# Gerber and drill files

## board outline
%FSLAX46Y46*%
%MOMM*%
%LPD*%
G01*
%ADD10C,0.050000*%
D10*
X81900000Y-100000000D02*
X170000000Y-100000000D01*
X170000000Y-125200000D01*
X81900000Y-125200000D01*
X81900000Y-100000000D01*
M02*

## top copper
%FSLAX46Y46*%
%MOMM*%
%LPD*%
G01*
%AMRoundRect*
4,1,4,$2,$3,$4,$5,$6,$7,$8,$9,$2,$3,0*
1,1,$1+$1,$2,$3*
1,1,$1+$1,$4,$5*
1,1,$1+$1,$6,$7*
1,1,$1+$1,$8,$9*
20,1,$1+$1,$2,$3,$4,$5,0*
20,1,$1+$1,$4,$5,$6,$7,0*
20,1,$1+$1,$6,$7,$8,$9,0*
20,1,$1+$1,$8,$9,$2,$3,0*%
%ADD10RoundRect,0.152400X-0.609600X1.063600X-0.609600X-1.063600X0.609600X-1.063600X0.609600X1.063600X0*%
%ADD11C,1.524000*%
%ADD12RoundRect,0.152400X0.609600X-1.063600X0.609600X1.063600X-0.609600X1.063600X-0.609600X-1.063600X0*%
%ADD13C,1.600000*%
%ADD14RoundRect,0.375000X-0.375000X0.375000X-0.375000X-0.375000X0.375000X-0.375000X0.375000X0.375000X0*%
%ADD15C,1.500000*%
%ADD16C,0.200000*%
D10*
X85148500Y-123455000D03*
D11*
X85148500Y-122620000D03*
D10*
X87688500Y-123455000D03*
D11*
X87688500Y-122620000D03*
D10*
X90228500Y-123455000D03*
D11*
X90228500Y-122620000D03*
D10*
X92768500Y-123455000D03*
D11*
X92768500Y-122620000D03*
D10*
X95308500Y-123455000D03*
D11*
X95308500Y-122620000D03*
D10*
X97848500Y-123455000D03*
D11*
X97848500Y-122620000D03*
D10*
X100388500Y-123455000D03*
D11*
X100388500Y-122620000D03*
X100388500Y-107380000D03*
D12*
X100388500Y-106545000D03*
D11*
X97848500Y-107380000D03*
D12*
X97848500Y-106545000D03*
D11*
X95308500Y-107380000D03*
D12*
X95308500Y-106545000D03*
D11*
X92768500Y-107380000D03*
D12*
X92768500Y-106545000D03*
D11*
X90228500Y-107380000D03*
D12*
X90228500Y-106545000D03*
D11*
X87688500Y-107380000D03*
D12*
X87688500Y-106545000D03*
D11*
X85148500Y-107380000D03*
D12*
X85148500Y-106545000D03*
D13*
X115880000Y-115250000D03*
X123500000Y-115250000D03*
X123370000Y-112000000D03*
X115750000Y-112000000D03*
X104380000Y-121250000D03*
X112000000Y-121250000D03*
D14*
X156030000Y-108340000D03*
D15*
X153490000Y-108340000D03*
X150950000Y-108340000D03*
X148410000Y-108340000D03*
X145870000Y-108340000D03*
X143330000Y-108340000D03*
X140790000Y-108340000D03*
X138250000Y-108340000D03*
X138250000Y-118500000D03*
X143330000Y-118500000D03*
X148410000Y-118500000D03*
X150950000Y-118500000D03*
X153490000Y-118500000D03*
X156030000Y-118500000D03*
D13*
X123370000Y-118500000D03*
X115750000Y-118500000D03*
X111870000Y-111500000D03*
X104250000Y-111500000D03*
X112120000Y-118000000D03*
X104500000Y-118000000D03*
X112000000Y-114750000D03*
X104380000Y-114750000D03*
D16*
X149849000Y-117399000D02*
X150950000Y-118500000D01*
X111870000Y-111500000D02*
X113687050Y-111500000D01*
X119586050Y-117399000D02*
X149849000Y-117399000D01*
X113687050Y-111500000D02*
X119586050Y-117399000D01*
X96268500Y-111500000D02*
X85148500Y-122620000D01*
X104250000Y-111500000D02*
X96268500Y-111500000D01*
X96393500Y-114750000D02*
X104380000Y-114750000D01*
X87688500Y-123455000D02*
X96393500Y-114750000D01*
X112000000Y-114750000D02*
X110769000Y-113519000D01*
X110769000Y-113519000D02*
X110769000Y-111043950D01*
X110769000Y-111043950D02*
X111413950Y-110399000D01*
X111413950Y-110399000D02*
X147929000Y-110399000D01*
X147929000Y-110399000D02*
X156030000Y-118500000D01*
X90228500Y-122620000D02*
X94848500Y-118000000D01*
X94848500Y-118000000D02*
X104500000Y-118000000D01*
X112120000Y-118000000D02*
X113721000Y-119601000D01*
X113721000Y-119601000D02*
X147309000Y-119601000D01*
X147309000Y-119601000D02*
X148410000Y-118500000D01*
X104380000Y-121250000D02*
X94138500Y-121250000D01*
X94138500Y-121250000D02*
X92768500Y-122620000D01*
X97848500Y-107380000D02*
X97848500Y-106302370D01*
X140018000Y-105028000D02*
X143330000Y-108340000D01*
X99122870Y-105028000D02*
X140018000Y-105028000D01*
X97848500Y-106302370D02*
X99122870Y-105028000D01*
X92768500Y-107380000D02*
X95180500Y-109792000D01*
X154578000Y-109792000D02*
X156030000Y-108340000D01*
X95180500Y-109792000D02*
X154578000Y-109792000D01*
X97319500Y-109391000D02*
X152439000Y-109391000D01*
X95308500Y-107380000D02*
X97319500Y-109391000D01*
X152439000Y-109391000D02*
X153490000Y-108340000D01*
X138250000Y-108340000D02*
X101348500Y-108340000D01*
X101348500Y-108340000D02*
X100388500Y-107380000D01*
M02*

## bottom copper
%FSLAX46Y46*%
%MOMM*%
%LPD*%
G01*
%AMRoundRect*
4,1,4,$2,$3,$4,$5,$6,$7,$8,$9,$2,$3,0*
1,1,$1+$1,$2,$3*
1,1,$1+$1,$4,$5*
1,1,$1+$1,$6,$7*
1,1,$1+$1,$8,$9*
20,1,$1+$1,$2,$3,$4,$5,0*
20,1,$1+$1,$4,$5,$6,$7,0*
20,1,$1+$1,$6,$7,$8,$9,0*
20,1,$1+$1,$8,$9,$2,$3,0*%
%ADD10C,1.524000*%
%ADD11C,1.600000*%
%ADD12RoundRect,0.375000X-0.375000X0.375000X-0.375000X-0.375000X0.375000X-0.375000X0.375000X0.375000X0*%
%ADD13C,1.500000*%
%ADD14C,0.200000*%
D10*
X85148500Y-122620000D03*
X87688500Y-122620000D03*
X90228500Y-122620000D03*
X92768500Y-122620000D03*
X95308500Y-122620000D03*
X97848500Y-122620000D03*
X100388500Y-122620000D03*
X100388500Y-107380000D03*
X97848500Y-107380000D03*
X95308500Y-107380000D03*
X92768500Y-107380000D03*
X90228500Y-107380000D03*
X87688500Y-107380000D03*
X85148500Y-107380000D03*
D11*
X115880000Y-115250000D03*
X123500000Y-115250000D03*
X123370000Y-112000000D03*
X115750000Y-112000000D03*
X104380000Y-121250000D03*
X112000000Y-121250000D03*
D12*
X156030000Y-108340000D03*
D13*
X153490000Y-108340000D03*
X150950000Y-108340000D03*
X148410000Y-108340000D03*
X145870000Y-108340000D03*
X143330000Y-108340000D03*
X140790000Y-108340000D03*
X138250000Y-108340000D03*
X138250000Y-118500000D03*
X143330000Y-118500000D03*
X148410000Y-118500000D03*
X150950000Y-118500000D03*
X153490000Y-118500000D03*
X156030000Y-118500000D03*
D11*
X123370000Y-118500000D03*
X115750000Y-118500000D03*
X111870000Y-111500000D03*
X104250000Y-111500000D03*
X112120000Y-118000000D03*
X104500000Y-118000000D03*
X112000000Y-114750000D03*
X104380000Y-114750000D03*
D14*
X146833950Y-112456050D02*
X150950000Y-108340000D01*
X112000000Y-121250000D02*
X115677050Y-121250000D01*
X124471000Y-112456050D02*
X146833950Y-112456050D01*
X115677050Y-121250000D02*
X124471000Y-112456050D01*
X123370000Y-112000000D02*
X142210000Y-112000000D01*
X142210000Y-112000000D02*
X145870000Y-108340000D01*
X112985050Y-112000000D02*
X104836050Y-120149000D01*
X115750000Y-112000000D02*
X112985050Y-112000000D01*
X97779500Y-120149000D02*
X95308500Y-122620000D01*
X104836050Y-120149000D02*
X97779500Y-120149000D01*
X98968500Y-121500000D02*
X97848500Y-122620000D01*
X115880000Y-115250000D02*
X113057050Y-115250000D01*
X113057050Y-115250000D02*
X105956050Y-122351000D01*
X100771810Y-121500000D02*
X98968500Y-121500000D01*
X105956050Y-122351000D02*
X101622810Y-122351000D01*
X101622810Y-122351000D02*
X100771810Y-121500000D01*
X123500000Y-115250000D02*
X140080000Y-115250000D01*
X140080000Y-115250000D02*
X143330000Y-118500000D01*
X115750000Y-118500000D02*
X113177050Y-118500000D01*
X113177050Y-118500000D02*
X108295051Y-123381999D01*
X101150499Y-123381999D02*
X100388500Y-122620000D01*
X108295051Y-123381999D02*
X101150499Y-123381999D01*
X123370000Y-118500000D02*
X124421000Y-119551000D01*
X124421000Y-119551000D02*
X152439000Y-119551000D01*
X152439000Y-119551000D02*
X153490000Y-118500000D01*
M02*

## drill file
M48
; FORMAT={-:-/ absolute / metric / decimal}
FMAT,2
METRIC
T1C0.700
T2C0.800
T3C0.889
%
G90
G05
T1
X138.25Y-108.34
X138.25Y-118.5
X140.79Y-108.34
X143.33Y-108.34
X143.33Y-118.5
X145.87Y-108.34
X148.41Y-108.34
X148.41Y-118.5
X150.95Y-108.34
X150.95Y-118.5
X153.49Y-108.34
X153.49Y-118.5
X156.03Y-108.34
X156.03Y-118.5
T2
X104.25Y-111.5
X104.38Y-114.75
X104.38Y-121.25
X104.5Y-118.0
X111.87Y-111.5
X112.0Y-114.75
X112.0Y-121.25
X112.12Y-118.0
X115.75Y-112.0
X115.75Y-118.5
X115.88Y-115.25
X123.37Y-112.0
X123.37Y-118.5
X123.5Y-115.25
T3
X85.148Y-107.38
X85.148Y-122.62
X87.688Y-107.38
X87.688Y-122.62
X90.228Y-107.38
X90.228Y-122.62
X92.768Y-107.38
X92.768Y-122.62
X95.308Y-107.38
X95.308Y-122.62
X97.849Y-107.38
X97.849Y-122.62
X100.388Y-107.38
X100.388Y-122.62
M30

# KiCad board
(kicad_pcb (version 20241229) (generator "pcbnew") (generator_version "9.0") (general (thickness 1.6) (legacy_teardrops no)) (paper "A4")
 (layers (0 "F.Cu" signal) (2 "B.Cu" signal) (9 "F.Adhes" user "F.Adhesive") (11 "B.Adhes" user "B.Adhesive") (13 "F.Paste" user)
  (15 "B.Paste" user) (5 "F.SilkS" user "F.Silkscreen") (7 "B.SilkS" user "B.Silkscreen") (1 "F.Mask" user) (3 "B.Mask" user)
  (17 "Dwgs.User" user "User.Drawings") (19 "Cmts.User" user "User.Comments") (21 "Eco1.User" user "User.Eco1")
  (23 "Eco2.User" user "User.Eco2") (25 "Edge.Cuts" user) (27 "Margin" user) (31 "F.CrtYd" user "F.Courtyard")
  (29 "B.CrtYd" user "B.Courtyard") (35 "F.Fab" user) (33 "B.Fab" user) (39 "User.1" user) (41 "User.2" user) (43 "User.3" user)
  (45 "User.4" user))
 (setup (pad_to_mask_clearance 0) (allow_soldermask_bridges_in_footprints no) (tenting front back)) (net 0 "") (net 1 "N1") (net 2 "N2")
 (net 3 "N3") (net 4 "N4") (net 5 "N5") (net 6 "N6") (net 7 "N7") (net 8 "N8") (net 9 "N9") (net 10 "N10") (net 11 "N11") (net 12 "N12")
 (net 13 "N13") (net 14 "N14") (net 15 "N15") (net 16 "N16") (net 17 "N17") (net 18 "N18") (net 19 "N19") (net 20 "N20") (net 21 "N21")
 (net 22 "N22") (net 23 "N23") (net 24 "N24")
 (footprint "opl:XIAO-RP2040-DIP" (layer "F.Cu") (at 92.7685 115 90)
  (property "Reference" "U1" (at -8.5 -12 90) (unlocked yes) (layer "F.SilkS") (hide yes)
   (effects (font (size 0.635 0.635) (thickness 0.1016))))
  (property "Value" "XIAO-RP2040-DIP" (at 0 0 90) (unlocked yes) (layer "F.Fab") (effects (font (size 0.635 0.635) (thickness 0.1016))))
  (pad "1" smd roundrect (at -8.455 -7.62 270) (size 2.432 1.524) (layers "F.Cu" "F.Mask") (roundrect_rratio 0.1) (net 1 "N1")
   (thermal_bridge_angle 45))
  (pad "1" thru_hole circle (at -7.62 -7.62 270) (size 1.524 1.524) (drill 0.889) (layers "*.Cu" "*.Mask") (remove_unused_layers no)
   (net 1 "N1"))
  (pad "2" smd roundrect (at -8.455 -5.08 270) (size 2.432 1.524) (layers "F.Cu" "F.Mask") (roundrect_rratio 0.1) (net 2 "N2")
   (thermal_bridge_angle 45))
  (pad "2" thru_hole circle (at -7.62 -5.08 270) (size 1.524 1.524) (drill 0.889) (layers "*.Cu" "*.Mask") (remove_unused_layers no)
   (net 2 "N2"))
  (pad "3" smd roundrect (at -8.455 -2.54 270) (size 2.432 1.524) (layers "F.Cu" "F.Mask") (roundrect_rratio 0.1) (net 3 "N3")
   (thermal_bridge_angle 45))
  (pad "3" thru_hole circle (at -7.62 -2.54 270) (size 1.524 1.524) (drill 0.889) (layers "*.Cu" "*.Mask") (remove_unused_layers no)
   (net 3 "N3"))
  (pad "4" smd roundrect (at -8.455 0 270) (size 2.432 1.524) (layers "F.Cu" "F.Mask") (roundrect_rratio 0.1) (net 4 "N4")
   (thermal_bridge_angle 45))
  (pad "4" thru_hole circle (at -7.62 0 270) (size 1.524 1.524) (drill 0.889) (layers "*.Cu" "*.Mask") (remove_unused_layers no)
   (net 4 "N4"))
  (pad "5" smd roundrect (at -8.455 2.54 270) (size 2.432 1.524) (layers "F.Cu" "F.Mask") (roundrect_rratio 0.1) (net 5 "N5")
   (thermal_bridge_angle 45))
  (pad "5" thru_hole circle (at -7.62 2.54 270) (size 1.524 1.524) (drill 0.889) (layers "*.Cu" "*.Mask") (remove_unused_layers no)
   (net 5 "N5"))
  (pad "6" smd roundrect (at -8.455 5.08 270) (size 2.432 1.524) (layers "F.Cu" "F.Mask") (roundrect_rratio 0.1) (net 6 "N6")
   (thermal_bridge_angle 45))
  (pad "6" thru_hole circle (at -7.62 5.08 270) (size 1.524 1.524) (drill 0.889) (layers "*.Cu" "*.Mask") (remove_unused_layers no)
   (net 6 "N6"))
  (pad "7" smd roundrect (at -8.455 7.62 270) (size 2.432 1.524) (layers "F.Cu" "F.Mask") (roundrect_rratio 0.1) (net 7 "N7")
   (thermal_bridge_angle 45))
  (pad "7" thru_hole circle (at -7.62 7.62 270) (size 1.524 1.524) (drill 0.889) (layers "*.Cu" "*.Mask") (remove_unused_layers no)
   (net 7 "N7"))
  (pad "8" thru_hole circle (at 7.62 7.62 90) (size 1.524 1.524) (drill 0.889) (layers "*.Cu" "*.Mask") (remove_unused_layers no)
   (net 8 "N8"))
  (pad "8" smd roundrect (at 8.455 7.62 90) (size 2.432 1.524) (layers "F.Cu" "F.Mask") (roundrect_rratio 0.1) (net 8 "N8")
   (thermal_bridge_angle 45))
  (pad "9" thru_hole circle (at 7.62 5.08 90) (size 1.524 1.524) (drill 0.889) (layers "*.Cu" "*.Mask") (remove_unused_layers no)
   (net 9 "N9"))
  (pad "9" smd roundrect (at 8.455 5.08 90) (size 2.432 1.524) (layers "F.Cu" "F.Mask") (roundrect_rratio 0.1) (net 9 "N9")
   (thermal_bridge_angle 45))
  (pad "10" thru_hole circle (at 7.62 2.54 90) (size 1.524 1.524) (drill 0.889) (layers "*.Cu" "*.Mask") (remove_unused_layers no)
   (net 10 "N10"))
  (pad "10" smd roundrect (at 8.455 2.54 90) (size 2.432 1.524) (layers "F.Cu" "F.Mask") (roundrect_rratio 0.1) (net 10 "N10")
   (thermal_bridge_angle 45))
  (pad "11" thru_hole circle (at 7.62 0 90) (size 1.524 1.524) (drill 0.889) (layers "*.Cu" "*.Mask") (remove_unused_layers no)
   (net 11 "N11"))
  (pad "11" smd roundrect (at 8.455 0 90) (size 2.432 1.524) (layers "F.Cu" "F.Mask") (roundrect_rratio 0.1) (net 11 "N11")
   (thermal_bridge_angle 45))
  (pad "12" thru_hole circle (at 7.62 -2.54 90) (size 1.524 1.524) (drill 0.889) (layers "*.Cu" "*.Mask") (remove_unused_layers no)
   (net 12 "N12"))
  (pad "12" smd roundrect (at 8.455 -2.54 90) (size 2.432 1.524) (layers "F.Cu" "F.Mask") (roundrect_rratio 0.1) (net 12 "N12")
   (thermal_bridge_angle 45))
  (pad "13" thru_hole circle (at 7.62 -5.08 90) (size 1.524 1.524) (drill 0.889) (layers "*.Cu" "*.Mask") (remove_unused_layers no)
   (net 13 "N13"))
  (pad "13" smd roundrect (at 8.455 -5.08 90) (size 2.432 1.524) (layers "F.Cu" "F.Mask") (roundrect_rratio 0.1) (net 13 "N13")
   (thermal_bridge_angle 45))
  (pad "14" thru_hole circle (at 7.62 -7.62 90) (size 1.524 1.524) (drill 0.889) (layers "*.Cu" "*.Mask") (remove_unused_layers no)
   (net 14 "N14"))
  (pad "14" smd roundrect (at 8.455 -7.62 90) (size 2.432 1.524) (layers "F.Cu" "F.Mask") (roundrect_rratio 0.1) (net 14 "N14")
   (thermal_bridge_angle 45)))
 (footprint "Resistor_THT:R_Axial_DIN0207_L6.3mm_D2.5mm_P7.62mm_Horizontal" (layer "F.Cu") (at 115.88 115.25)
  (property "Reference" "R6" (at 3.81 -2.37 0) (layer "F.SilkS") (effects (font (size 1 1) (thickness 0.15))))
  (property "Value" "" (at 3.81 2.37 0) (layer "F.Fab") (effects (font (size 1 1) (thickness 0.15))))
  (pad "1" thru_hole circle (at 0 0) (size 1.6 1.6) (drill 0.8) (layers "*.Cu" "*.Mask") (remove_unused_layers no) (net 6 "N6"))
  (pad "2" thru_hole circle (at 7.62 0) (size 1.6 1.6) (drill 0.8) (layers "*.Cu" "*.Mask") (remove_unused_layers no) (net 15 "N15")))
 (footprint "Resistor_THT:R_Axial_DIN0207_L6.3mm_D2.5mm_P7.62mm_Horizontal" (layer "F.Cu") (at 123.37 112 180)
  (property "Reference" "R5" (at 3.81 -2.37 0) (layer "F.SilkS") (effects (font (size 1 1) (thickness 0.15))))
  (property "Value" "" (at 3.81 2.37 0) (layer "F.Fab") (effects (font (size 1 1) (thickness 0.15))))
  (pad "1" thru_hole circle (at 0 0 180) (size 1.6 1.6) (drill 0.8) (layers "*.Cu" "*.Mask") (remove_unused_layers no) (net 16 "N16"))
  (pad "2" thru_hole circle (at 7.62 0 180) (size 1.6 1.6) (drill 0.8) (layers "*.Cu" "*.Mask") (remove_unused_layers no) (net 5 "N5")))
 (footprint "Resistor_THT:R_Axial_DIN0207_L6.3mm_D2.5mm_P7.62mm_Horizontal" (layer "F.Cu") (at 104.38 121.25)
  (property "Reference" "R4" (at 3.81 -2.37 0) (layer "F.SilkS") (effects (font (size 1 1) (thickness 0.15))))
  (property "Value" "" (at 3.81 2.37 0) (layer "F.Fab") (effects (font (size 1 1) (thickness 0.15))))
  (pad "1" thru_hole circle (at 0 0) (size 1.6 1.6) (drill 0.8) (layers "*.Cu" "*.Mask") (remove_unused_layers no) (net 4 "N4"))
  (pad "2" thru_hole circle (at 7.62 0) (size 1.6 1.6) (drill 0.8) (layers "*.Cu" "*.Mask") (remove_unused_layers no) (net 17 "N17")))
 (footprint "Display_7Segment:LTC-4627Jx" (layer "F.Cu") (at 156.03 108.34 -90)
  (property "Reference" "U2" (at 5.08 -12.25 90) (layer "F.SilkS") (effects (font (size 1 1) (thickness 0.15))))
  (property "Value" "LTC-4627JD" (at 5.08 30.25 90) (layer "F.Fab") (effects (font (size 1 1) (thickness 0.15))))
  (pad "1" thru_hole roundrect (at 0 0 270) (size 1.5 1.5) (drill 0.7) (layers "*.Cu" "*.Mask") (remove_unused_layers no)
   (roundrect_rratio 0.25) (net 11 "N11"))
  (pad "2" thru_hole circle (at 0 2.54 270) (size 1.5 1.5) (drill 0.7) (layers "*.Cu" "*.Mask") (remove_unused_layers no) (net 10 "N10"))
  (pad "3" thru_hole circle (at 0 5.08 270) (size 1.5 1.5) (drill 0.7) (layers "*.Cu" "*.Mask") (remove_unused_layers no) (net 17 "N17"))
  (pad "4" thru_hole circle (at 0 7.62 270) (size 1.5 1.5) (drill 0.7) (layers "*.Cu" "*.Mask") (remove_unused_layers no) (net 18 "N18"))
  (pad "5" thru_hole circle (at 0 10.16 270) (size 1.5 1.5) (drill 0.7) (layers "*.Cu" "*.Mask") (remove_unused_layers no) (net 16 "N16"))
  (pad "6" thru_hole circle (at 0 12.7 270) (size 1.5 1.5) (drill 0.7) (layers "*.Cu" "*.Mask") (remove_unused_layers no) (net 9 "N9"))
  (pad "7" thru_hole circle (at 0 15.24 270) (size 1.5 1.5) (drill 0.7) (layers "*.Cu" "*.Mask") (remove_unused_layers no) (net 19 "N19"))
  (pad "8" thru_hole circle (at 0 17.78 270) (size 1.5 1.5) (drill 0.7) (layers "*.Cu" "*.Mask") (remove_unused_layers no) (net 8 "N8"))
  (pad "9" thru_hole circle (at 10.16 17.78 270) (size 1.5 1.5) (drill 0.7) (layers "*.Cu" "*.Mask") (remove_unused_layers no)
   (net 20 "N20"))
  (pad "11" thru_hole circle (at 10.16 12.7 270) (size 1.5 1.5) (drill 0.7) (layers "*.Cu" "*.Mask") (remove_unused_layers no)
   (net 15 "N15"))
  (pad "13" thru_hole circle (at 10.16 7.62 270) (size 1.5 1.5) (drill 0.7) (layers "*.Cu" "*.Mask") (remove_unused_layers no)
   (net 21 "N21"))
  (pad "14" thru_hole circle (at 10.16 5.08 270) (size 1.5 1.5) (drill 0.7) (layers "*.Cu" "*.Mask") (remove_unused_layers no)
   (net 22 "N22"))
  (pad "15" thru_hole circle (at 10.16 2.54 270) (size 1.5 1.5) (drill 0.7) (layers "*.Cu" "*.Mask") (remove_unused_layers no)
   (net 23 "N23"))
  (pad "16" thru_hole circle (at 10.16 0 270) (size 1.5 1.5) (drill 0.7) (layers "*.Cu" "*.Mask") (remove_unused_layers no) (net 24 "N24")))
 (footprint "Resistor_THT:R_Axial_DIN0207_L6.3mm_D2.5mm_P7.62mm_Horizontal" (layer "F.Cu") (at 123.37 118.5 180)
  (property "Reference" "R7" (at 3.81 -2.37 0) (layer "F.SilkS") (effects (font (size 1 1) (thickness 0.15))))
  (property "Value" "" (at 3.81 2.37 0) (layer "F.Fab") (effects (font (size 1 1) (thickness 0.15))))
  (pad "1" thru_hole circle (at 0 0 180) (size 1.6 1.6) (drill 0.8) (layers "*.Cu" "*.Mask") (remove_unused_layers no) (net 23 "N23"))
  (pad "2" thru_hole circle (at 7.62 0 180) (size 1.6 1.6) (drill 0.8) (layers "*.Cu" "*.Mask") (remove_unused_layers no) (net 7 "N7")))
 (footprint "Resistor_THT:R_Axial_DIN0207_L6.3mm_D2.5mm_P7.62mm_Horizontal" (layer "B.Cu") (at 111.87 111.5 180)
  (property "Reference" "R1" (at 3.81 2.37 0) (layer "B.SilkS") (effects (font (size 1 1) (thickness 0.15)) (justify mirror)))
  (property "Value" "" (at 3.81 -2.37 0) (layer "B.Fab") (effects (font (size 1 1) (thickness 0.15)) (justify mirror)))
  (pad "1" thru_hole circle (at 0 0 180) (size 1.6 1.6) (drill 0.8) (layers "*.Cu" "*.Mask") (remove_unused_layers no) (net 22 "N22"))
  (pad "2" thru_hole circle (at 7.62 0 180) (size 1.6 1.6) (drill 0.8) (layers "*.Cu" "*.Mask") (remove_unused_layers no) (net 1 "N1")))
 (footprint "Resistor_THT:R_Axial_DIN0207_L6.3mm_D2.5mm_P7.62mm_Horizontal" (layer "B.Cu") (at 112.12 118 180)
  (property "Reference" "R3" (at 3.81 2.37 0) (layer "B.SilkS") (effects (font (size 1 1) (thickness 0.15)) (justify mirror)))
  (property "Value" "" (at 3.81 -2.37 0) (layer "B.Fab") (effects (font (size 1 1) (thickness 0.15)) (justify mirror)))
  (pad "1" thru_hole circle (at 0 0 180) (size 1.6 1.6) (drill 0.8) (layers "*.Cu" "*.Mask") (remove_unused_layers no) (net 21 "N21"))
  (pad "2" thru_hole circle (at 7.62 0 180) (size 1.6 1.6) (drill 0.8) (layers "*.Cu" "*.Mask") (remove_unused_layers no) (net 3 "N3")))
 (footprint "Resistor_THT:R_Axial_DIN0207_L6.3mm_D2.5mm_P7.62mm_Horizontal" (layer "B.Cu") (at 112 114.75 180)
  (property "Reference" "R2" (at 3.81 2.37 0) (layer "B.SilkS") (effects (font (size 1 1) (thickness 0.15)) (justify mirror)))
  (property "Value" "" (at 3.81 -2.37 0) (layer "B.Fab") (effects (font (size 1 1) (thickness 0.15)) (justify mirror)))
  (pad "1" thru_hole circle (at 0 0 180) (size 1.6 1.6) (drill 0.8) (layers "*.Cu" "*.Mask") (remove_unused_layers no) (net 24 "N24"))
  (pad "2" thru_hole circle (at 7.62 0 180) (size 1.6 1.6) (drill 0.8) (layers "*.Cu" "*.Mask") (remove_unused_layers no) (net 2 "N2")))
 (gr_rect (start 81.9 100) (end 170 125.2) (stroke (width 0.05) (type default)) (fill no) (layer "Edge.Cuts"))
 (segment (start 149.849 117.399) (end 150.95 118.5) (width 0.2) (layer "F.Cu") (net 22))
 (segment (start 111.87 111.5) (end 113.68705 111.5) (width 0.2) (layer "F.Cu") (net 22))
 (segment (start 119.58605 117.399) (end 149.849 117.399) (width 0.2) (layer "F.Cu") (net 22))
 (segment (start 113.68705 111.5) (end 119.58605 117.399) (width 0.2) (layer "F.Cu") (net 22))
 (segment (start 96.2685 111.5) (end 85.1485 122.62) (width 0.2) (layer "F.Cu") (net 1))
 (segment (start 104.25 111.5) (end 96.2685 111.5) (width 0.2) (layer "F.Cu") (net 1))
 (segment (start 96.3935 114.75) (end 104.38 114.75) (width 0.2) (layer "F.Cu") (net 2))
 (segment (start 87.6885 123.455) (end 96.3935 114.75) (width 0.2) (layer "F.Cu") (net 2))
 (segment (start 112 114.75) (end 110.769 113.519) (width 0.2) (layer "F.Cu") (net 24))
 (segment (start 110.769 113.519) (end 110.769 111.04395) (width 0.2) (layer "F.Cu") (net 24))
 (segment (start 110.769 111.04395) (end 111.41395 110.399) (width 0.2) (layer "F.Cu") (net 24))
 (segment (start 111.41395 110.399) (end 147.929 110.399) (width 0.2) (layer "F.Cu") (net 24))
 (segment (start 147.929 110.399) (end 156.03 118.5) (width 0.2) (layer "F.Cu") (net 24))
 (segment (start 90.2285 122.62) (end 94.8485 118) (width 0.2) (layer "F.Cu") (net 3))
 (segment (start 94.8485 118) (end 104.5 118) (width 0.2) (layer "F.Cu") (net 3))
 (segment (start 112.12 118) (end 113.721 119.601) (width 0.2) (layer "F.Cu") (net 21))
 (segment (start 113.721 119.601) (end 147.309 119.601) (width 0.2) (layer "F.Cu") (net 21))
 (segment (start 147.309 119.601) (end 148.41 118.5) (width 0.2) (layer "F.Cu") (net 21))
 (segment (start 146.83395 112.45605) (end 150.95 108.34) (width 0.2) (layer "B.Cu") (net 17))
 (segment (start 112 121.25) (end 115.67705 121.25) (width 0.2) (layer "B.Cu") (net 17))
 (segment (start 124.471 112.45605) (end 146.83395 112.45605) (width 0.2) (layer "B.Cu") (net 17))
 (segment (start 115.67705 121.25) (end 124.471 112.45605) (width 0.2) (layer "B.Cu") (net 17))
 (segment (start 104.38 121.25) (end 94.1385 121.25) (width 0.2) (layer "F.Cu") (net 4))
 (segment (start 94.1385 121.25) (end 92.7685 122.62) (width 0.2) (layer "F.Cu") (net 4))
 (segment (start 123.37 112) (end 142.21 112) (width 0.2) (layer "B.Cu") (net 16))
 (segment (start 142.21 112) (end 145.87 108.34) (width 0.2) (layer "B.Cu") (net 16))
 (segment (start 112.98505 112) (end 104.83605 120.149) (width 0.2) (layer "B.Cu") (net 5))
 (segment (start 115.75 112) (end 112.98505 112) (width 0.2) (layer "B.Cu") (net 5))
 (segment (start 97.7795 120.149) (end 95.3085 122.62) (width 0.2) (layer "B.Cu") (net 5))
 (segment (start 104.83605 120.149) (end 97.7795 120.149) (width 0.2) (layer "B.Cu") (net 5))
 (segment (start 98.9685 121.5) (end 97.8485 122.62) (width 0.2) (layer "B.Cu") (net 6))
 (segment (start 115.88 115.25) (end 113.05705 115.25) (width 0.2) (layer "B.Cu") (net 6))
 (segment (start 113.05705 115.25) (end 105.95605 122.351) (width 0.2) (layer "B.Cu") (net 6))
 (segment (start 100.77181 121.5) (end 98.9685 121.5) (width 0.2) (layer "B.Cu") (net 6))
 (segment (start 105.95605 122.351) (end 101.62281 122.351) (width 0.2) (layer "B.Cu") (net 6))
 (segment (start 101.62281 122.351) (end 100.77181 121.5) (width 0.2) (layer "B.Cu") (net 6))
 (segment (start 123.5 115.25) (end 140.08 115.25) (width 0.2) (layer "B.Cu") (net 15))
 (segment (start 140.08 115.25) (end 143.33 118.5) (width 0.2) (layer "B.Cu") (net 15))
 (segment (start 115.75 118.5) (end 113.17705 118.5) (width 0.2) (layer "B.Cu") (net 7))
 (segment (start 113.17705 118.5) (end 108.295051 123.381999) (width 0.2) (layer "B.Cu") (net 7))
 (segment (start 101.150499 123.381999) (end 100.3885 122.62) (width 0.2) (layer "B.Cu") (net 7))
 (segment (start 108.295051 123.381999) (end 101.150499 123.381999) (width 0.2) (layer "B.Cu") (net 7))
 (segment (start 123.37 118.5) (end 124.421 119.551) (width 0.2) (layer "B.Cu") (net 23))
 (segment (start 124.421 119.551) (end 152.439 119.551) (width 0.2) (layer "B.Cu") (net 23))
 (segment (start 152.439 119.551) (end 153.49 118.5) (width 0.2) (layer "B.Cu") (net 23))
 (segment (start 97.8485 107.38) (end 97.8485 106.30237) (width 0.2) (layer "F.Cu") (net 9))
 (segment (start 140.018 105.028) (end 143.33 108.34) (width 0.2) (layer "F.Cu") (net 9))
 (segment (start 99.12287 105.028) (end 140.018 105.028) (width 0.2) (layer "F.Cu") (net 9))
 (segment (start 97.8485 106.30237) (end 99.12287 105.028) (width 0.2) (layer "F.Cu") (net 9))
 (segment (start 92.7685 107.38) (end 95.1805 109.792) (width 0.2) (layer "F.Cu") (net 11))
 (segment (start 154.578 109.792) (end 156.03 108.34) (width 0.2) (layer "F.Cu") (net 11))
 (segment (start 95.1805 109.792) (end 154.578 109.792) (width 0.2) (layer "F.Cu") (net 11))
 (segment (start 97.3195 109.391) (end 152.439 109.391) (width 0.2) (layer "F.Cu") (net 10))
 (segment (start 95.3085 107.38) (end 97.3195 109.391) (width 0.2) (layer "F.Cu") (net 10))
 (segment (start 152.439 109.391) (end 153.49 108.34) (width 0.2) (layer "F.Cu") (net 10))
 (segment (start 138.25 108.34) (end 101.3485 108.34) (width 0.2) (layer "F.Cu") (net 8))
 (segment (start 101.3485 108.34) (end 100.3885 107.38) (width 0.2) (layer "F.Cu") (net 8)))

